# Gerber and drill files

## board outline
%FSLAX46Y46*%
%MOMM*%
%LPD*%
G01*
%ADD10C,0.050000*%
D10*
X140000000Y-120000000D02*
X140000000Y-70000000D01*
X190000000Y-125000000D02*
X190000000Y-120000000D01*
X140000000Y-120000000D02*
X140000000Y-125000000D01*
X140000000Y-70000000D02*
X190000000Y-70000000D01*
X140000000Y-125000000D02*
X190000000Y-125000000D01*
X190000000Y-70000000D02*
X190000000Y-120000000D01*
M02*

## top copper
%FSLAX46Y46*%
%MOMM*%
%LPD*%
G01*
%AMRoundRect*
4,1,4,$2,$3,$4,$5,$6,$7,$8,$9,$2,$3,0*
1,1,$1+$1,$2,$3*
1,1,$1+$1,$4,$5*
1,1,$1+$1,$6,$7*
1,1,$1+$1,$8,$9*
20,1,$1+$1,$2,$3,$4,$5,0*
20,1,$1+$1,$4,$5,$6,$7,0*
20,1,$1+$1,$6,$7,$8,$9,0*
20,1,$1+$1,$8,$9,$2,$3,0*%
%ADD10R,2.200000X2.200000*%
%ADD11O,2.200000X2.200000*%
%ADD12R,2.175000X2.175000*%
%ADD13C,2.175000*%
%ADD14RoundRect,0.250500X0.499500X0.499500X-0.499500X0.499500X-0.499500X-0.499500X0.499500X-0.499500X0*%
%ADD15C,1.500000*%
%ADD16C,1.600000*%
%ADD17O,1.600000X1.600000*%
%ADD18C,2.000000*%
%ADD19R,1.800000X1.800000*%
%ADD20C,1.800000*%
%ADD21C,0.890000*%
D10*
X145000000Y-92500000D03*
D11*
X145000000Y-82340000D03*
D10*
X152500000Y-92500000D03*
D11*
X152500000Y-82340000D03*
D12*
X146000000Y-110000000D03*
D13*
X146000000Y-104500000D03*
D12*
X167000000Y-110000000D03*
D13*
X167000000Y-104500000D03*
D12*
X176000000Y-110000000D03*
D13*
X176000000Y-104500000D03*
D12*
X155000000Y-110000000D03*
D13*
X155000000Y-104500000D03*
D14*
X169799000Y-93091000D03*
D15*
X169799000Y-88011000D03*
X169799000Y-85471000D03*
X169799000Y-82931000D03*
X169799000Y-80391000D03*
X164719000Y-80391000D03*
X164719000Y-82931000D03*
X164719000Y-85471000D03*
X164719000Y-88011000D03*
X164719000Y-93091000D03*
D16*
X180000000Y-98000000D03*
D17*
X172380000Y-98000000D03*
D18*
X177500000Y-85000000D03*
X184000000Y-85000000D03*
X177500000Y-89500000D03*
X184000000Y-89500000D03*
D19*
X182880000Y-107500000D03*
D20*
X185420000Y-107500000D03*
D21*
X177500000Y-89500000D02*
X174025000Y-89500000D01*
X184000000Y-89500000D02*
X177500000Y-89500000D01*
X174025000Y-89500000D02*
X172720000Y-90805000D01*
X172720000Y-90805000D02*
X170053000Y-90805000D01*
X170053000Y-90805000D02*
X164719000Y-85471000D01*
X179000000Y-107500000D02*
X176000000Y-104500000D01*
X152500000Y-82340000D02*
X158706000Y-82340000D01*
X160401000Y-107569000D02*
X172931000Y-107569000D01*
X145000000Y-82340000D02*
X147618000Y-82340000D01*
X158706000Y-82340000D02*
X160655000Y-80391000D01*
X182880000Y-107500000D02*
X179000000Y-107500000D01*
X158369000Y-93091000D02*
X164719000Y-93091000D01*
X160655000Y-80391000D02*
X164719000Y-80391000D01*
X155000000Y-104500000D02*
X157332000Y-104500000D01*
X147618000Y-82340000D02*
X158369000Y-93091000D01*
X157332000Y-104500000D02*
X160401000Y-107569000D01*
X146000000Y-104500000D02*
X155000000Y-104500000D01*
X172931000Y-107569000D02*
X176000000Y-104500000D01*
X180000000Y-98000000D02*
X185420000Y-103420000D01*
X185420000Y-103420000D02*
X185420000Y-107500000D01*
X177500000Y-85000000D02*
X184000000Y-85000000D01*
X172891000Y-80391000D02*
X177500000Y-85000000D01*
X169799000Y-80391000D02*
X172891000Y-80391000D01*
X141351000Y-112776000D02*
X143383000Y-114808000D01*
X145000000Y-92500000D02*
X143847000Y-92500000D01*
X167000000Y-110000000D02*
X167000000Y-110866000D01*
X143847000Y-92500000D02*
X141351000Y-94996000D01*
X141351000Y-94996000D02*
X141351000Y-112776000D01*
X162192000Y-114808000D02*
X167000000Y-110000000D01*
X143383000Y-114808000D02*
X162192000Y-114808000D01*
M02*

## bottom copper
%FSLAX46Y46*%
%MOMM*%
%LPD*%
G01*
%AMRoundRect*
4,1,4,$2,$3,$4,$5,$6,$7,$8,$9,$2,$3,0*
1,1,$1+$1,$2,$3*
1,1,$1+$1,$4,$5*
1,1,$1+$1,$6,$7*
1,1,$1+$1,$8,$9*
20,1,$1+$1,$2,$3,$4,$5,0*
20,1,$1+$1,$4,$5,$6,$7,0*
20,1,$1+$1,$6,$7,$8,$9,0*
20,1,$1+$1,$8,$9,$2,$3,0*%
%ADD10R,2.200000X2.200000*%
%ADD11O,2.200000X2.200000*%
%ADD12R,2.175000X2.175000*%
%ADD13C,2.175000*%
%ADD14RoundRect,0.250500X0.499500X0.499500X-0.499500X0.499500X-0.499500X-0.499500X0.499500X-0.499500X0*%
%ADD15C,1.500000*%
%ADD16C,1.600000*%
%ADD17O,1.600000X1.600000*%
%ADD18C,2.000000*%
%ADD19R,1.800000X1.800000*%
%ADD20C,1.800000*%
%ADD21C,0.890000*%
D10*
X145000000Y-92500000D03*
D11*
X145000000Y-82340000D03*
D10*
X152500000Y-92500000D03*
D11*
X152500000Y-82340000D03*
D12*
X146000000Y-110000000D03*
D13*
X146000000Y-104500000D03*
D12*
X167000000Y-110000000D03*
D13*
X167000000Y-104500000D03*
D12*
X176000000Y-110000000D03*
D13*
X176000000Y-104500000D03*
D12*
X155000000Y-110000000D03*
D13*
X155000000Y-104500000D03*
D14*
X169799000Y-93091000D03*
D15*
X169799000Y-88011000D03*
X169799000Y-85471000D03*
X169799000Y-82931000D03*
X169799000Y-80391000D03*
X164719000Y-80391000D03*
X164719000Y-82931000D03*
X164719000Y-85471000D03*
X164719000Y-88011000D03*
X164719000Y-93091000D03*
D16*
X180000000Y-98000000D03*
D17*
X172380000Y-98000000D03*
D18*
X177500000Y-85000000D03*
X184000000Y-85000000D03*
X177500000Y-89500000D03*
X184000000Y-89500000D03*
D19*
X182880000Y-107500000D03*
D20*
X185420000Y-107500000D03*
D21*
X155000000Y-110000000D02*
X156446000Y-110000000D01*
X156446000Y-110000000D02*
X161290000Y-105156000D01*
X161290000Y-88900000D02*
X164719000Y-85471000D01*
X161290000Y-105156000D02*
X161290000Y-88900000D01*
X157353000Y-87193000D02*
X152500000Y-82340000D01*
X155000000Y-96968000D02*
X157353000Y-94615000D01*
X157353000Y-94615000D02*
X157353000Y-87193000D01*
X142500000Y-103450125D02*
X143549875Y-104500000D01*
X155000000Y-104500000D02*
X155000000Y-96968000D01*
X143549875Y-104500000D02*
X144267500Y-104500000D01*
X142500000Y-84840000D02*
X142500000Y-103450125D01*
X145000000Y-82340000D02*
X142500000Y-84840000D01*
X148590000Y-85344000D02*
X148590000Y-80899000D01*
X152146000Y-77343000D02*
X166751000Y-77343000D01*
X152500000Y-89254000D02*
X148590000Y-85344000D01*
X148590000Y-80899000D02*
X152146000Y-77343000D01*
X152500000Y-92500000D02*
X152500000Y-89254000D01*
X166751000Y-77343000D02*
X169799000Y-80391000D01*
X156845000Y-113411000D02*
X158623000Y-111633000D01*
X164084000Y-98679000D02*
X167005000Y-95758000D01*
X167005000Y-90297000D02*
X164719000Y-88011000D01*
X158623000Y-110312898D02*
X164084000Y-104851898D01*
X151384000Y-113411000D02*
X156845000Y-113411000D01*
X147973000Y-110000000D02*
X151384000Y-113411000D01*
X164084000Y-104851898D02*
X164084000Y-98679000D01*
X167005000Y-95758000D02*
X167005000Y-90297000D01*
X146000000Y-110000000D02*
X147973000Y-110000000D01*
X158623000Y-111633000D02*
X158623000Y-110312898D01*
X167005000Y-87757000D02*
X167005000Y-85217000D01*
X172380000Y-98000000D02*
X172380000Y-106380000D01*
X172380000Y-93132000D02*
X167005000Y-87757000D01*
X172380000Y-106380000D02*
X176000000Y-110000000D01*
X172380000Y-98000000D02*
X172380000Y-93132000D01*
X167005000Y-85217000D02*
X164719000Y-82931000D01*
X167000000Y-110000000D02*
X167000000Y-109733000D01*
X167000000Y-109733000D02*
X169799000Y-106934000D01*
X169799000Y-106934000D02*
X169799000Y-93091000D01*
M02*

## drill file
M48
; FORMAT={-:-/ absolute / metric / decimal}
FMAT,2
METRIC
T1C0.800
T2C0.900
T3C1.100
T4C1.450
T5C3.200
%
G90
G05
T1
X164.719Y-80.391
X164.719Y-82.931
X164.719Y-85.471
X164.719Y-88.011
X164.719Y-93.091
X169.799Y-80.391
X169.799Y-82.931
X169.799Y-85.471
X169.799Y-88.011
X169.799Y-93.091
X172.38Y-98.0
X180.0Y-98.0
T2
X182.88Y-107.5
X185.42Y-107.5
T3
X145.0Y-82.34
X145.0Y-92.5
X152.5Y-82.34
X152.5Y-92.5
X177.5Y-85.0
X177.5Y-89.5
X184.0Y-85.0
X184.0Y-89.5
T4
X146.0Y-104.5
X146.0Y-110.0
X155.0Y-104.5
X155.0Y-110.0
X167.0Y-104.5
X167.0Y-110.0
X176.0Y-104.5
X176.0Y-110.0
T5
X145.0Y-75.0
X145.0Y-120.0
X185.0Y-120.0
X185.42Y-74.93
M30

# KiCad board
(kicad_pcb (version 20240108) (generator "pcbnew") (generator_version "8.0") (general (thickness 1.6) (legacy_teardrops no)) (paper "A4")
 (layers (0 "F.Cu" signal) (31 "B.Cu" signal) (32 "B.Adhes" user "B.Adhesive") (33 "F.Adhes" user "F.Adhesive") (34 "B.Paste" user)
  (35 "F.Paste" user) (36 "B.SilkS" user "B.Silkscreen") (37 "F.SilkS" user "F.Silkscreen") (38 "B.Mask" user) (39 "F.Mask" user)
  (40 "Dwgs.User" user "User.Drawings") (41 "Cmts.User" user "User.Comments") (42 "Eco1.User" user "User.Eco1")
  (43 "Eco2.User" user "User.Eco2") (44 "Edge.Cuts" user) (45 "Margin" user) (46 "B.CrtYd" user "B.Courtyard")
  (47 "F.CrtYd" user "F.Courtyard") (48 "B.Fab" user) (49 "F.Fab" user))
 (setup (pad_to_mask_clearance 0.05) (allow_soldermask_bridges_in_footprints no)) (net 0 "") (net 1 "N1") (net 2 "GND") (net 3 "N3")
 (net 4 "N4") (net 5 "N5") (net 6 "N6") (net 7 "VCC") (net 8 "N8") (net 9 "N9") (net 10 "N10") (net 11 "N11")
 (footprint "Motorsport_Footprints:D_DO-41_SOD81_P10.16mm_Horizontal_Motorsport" (layer "F.Cu") (at 145 92.5 90)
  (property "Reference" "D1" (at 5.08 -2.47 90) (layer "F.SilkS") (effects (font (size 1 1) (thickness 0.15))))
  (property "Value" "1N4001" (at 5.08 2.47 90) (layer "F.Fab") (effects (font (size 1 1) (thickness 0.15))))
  (pad "1" thru_hole rect (at 0 0 90) (size 2.2 2.2) (drill 1.1) (layers "*.Cu" "*.Mask") (remove_unused_layers no) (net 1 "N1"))
  (pad "2" thru_hole oval (at 10.16 0 90) (size 2.2 2.2) (drill 1.1) (layers "*.Cu" "*.Mask") (remove_unused_layers no) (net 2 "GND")))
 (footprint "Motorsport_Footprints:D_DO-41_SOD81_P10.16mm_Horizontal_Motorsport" (layer "F.Cu") (at 152.5 92.5 90)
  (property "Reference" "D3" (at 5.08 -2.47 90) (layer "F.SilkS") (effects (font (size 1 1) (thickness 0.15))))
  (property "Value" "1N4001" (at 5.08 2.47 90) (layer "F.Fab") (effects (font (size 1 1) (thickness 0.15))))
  (pad "1" thru_hole rect (at 0 0 90) (size 2.2 2.2) (drill 1.1) (layers "*.Cu" "*.Mask") (remove_unused_layers no) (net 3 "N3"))
  (pad "2" thru_hole oval (at 10.16 0 90) (size 2.2 2.2) (drill 1.1) (layers "*.Cu" "*.Mask") (remove_unused_layers no) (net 2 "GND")))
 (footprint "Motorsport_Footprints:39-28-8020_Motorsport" (layer "F.Cu") (at 146 110)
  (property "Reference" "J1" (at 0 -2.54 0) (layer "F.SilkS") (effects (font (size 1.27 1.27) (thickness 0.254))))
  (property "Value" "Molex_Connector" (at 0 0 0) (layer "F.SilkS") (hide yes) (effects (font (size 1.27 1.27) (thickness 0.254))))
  (pad "1" thru_hole rect (at 0 0) (size 2.175 2.175) (drill 1.45) (layers "*.Cu" "*.Mask") (remove_unused_layers no) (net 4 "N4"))
  (pad "2" thru_hole circle (at 0 -5.5) (size 2.175 2.175) (drill 1.45) (layers "*.Cu" "*.Mask") (remove_unused_layers no) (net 2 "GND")))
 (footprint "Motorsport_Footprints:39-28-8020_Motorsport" (layer "F.Cu") (at 167 110)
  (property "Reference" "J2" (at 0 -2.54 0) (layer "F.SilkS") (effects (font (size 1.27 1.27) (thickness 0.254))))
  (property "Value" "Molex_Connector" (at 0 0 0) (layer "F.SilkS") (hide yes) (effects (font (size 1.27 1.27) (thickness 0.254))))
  (pad "1" thru_hole rect (at 0 0) (size 2.175 2.175) (drill 1.45) (layers "*.Cu" "*.Mask") (remove_unused_layers no) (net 1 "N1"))
  (pad "2" thru_hole circle (at 0 -5.5) (size 2.175 2.175) (drill 1.45) (layers "*.Cu" "*.Mask") (remove_unused_layers no) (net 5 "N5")))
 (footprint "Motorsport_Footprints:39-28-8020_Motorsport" (layer "F.Cu") (at 176 110)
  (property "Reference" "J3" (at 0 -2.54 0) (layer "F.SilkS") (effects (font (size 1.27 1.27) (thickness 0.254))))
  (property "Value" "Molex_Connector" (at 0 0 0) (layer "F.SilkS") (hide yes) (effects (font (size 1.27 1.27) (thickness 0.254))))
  (pad "1" thru_hole rect (at 0 0) (size 2.175 2.175) (drill 1.45) (layers "*.Cu" "*.Mask") (remove_unused_layers no) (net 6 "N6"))
  (pad "2" thru_hole circle (at 0 -5.5) (size 2.175 2.175) (drill 1.45) (layers "*.Cu" "*.Mask") (remove_unused_layers no) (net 2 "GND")))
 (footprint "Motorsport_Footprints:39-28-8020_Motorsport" (layer "F.Cu") (at 155 110)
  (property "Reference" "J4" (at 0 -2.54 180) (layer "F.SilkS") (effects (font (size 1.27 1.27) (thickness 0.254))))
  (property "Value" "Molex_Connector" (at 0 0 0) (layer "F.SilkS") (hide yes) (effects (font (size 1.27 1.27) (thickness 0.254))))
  (pad "1" thru_hole rect (at 0 0) (size 2.175 2.175) (drill 1.45) (layers "*.Cu" "*.Mask") (remove_unused_layers no) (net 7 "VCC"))
  (pad "2" thru_hole circle (at 0 -5.5) (size 2.175 2.175) (drill 1.45) (layers "*.Cu" "*.Mask") (remove_unused_layers no) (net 2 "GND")))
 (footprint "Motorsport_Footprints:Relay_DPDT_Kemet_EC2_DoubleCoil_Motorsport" (layer "F.Cu") (at 165.989 85.471 180)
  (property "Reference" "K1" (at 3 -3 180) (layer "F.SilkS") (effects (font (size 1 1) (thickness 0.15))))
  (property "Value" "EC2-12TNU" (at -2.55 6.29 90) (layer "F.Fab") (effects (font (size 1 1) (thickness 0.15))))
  (pad "1" thru_hole roundrect (at -3.81 -7.62 180) (size 1.5 1.5) (drill 0.8) (layers "*.Cu" "*.Mask") (remove_unused_layers no)
   (roundrect_rratio 0.167) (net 1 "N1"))
  (pad "3" thru_hole circle (at -3.81 -2.54 180) (size 1.5 1.5) (drill 0.8) (layers "*.Cu" "*.Mask") (remove_unused_layers no) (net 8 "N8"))
  (pad "4" thru_hole circle (at -3.81 0 180) (size 1.5 1.5) (drill 0.8) (layers "*.Cu" "*.Mask") (remove_unused_layers no) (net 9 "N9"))
  (pad "5" thru_hole circle (at -3.81 2.54 180) (size 1.5 1.5) (drill 0.8) (layers "*.Cu" "*.Mask") (remove_unused_layers no) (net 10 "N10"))
  (pad "6" thru_hole circle (at -3.81 5.08 180) (size 1.5 1.5) (drill 0.8) (layers "*.Cu" "*.Mask") (remove_unused_layers no) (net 3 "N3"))
  (pad "7" thru_hole circle (at 1.27 5.08 180) (size 1.5 1.5) (drill 0.8) (layers "*.Cu" "*.Mask") (remove_unused_layers no) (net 2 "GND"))
  (pad "8" thru_hole circle (at 1.27 2.54 180) (size 1.5 1.5) (drill 0.8) (layers "*.Cu" "*.Mask") (remove_unused_layers no) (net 6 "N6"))
  (pad "9" thru_hole circle (at 1.27 0 180) (size 1.5 1.5) (drill 0.8) (layers "*.Cu" "*.Mask") (remove_unused_layers no) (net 7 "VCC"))
  (pad "10" thru_hole circle (at 1.27 -2.54 180) (size 1.5 1.5) (drill 0.8) (layers "*.Cu" "*.Mask") (remove_unused_layers no) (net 4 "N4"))
  (pad "12" thru_hole circle (at 1.27 -7.62 180) (size 1.5 1.5) (drill 0.8) (layers "*.Cu" "*.Mask") (remove_unused_layers no) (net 2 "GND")))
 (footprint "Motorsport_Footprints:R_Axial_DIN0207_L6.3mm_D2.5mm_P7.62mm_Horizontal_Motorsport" (layer "F.Cu") (at 180 98 180)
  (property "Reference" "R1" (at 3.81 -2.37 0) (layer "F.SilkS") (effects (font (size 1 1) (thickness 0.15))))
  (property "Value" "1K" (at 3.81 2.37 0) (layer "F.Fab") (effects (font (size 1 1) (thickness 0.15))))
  (pad "1" thru_hole circle (at 0 0 180) (size 1.6 1.6) (drill 0.8) (layers "*.Cu" "*.Mask") (remove_unused_layers no) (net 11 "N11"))
  (pad "2" thru_hole oval (at 7.62 0 180) (size 1.6 1.6) (drill 0.8) (layers "*.Cu" "*.Mask") (remove_unused_layers no) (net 6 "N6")))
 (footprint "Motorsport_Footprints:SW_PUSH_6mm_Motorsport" (layer "F.Cu") (at 177.5 85)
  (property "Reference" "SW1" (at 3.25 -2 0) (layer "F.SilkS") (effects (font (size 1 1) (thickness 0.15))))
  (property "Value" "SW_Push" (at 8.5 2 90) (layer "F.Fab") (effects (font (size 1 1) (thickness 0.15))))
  (pad "1" thru_hole circle (at 0 0 90) (size 2 2) (drill 1.1) (layers "*.Cu" "*.Mask") (remove_unused_layers no) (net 3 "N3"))
  (pad "1" thru_hole circle (at 6.5 0 90) (size 2 2) (drill 1.1) (layers "*.Cu" "*.Mask") (remove_unused_layers no) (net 3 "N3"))
  (pad "2" thru_hole circle (at 0 4.5 90) (size 2 2) (drill 1.1) (layers "*.Cu" "*.Mask") (remove_unused_layers no) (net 7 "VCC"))
  (pad "2" thru_hole circle (at 6.5 4.5 90) (size 2 2) (drill 1.1) (layers "*.Cu" "*.Mask") (remove_unused_layers no) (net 7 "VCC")))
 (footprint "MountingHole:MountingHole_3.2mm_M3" (layer "F.Cu") (at 185.42 74.93)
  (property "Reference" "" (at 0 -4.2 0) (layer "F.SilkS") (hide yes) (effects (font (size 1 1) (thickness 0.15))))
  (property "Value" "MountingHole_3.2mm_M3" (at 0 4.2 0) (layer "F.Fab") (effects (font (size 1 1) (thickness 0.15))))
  (pad "" np_thru_hole circle (at 0 0) (size 3.2 3.2) (drill 3.2) (layers "*.Cu" "*.Mask")))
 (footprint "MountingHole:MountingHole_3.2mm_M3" (layer "F.Cu") (at 145 75)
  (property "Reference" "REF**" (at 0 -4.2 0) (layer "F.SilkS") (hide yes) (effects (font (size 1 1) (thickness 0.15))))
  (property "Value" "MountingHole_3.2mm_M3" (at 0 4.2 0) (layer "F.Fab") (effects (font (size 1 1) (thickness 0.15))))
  (pad "" np_thru_hole circle (at 0 0) (size 3.2 3.2) (drill 3.2) (layers "*.Cu" "*.Mask")))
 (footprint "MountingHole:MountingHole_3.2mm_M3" (layer "F.Cu") (at 145 120)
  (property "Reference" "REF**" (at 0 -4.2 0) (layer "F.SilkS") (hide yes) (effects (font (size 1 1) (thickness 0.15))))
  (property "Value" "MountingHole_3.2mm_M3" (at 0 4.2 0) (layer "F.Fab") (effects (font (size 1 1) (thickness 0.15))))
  (pad "" np_thru_hole circle (at 0 0) (size 3.2 3.2) (drill 3.2) (layers "*.Cu" "*.Mask")))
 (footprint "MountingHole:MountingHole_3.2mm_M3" (layer "F.Cu") (at 185 120)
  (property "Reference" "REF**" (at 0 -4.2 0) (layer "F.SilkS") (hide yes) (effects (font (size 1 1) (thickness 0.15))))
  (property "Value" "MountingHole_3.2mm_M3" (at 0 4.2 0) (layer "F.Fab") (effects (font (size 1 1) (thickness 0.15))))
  (pad "" np_thru_hole circle (at 0 0) (size 3.2 3.2) (drill 3.2) (layers "*.Cu" "*.Mask")))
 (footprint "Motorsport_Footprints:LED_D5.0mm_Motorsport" (layer "F.Cu") (at 182.88 107.5)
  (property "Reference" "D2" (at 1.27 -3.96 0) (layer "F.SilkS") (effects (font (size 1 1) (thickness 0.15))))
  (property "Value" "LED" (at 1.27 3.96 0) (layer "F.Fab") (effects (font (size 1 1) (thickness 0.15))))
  (pad "1" thru_hole rect (at 0 0) (size 1.8 1.8) (drill 0.9) (layers "*.Cu" "*.Mask") (remove_unused_layers no) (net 2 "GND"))
  (pad "2" thru_hole circle (at 2.54 0) (size 1.8 1.8) (drill 0.9) (layers "*.Cu" "*.Mask") (remove_unused_layers no) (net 11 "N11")))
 (gr_line (start 140 120) (end 140 70) (stroke (width 0.05) (type solid)) (layer "Edge.Cuts"))
 (gr_line (start 190 125) (end 190 120) (stroke (width 0.05) (type solid)) (layer "Edge.Cuts"))
 (gr_line (start 140 120) (end 140 125) (stroke (width 0.05) (type solid)) (layer "Edge.Cuts"))
 (gr_line (start 140 70) (end 190 70) (stroke (width 0.05) (type solid)) (layer "Edge.Cuts"))
 (gr_line (start 140 125) (end 190 125) (stroke (width 0.05) (type solid)) (layer "Edge.Cuts"))
 (gr_line (start 190 70) (end 190 120) (stroke (width 0.05) (type solid)) (layer "Edge.Cuts"))
 (segment (start 177.5 89.5) (end 174.025 89.5) (width 0.89) (layer "F.Cu") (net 7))
 (segment (start 184 89.5) (end 177.5 89.5) (width 0.89) (layer "F.Cu") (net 7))
 (segment (start 174.025 89.5) (end 172.72 90.805) (width 0.89) (layer "F.Cu") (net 7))
 (segment (start 172.72 90.805) (end 170.053 90.805) (width 0.89) (layer "F.Cu") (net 7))
 (segment (start 170.053 90.805) (end 164.719 85.471) (width 0.89) (layer "F.Cu") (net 7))
 (segment (start 155 110) (end 156.446 110) (width 0.89) (layer "B.Cu") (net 7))
 (segment (start 156.446 110) (end 161.29 105.156) (width 0.89) (layer "B.Cu") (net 7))
 (segment (start 161.29 88.9) (end 164.719 85.471) (width 0.89) (layer "B.Cu") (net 7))
 (segment (start 161.29 105.156) (end 161.29 88.9) (width 0.89) (layer "B.Cu") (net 7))
 (segment (start 179 107.5) (end 176 104.5) (width 0.89) (layer "F.Cu") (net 2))
 (segment (start 152.5 82.34) (end 158.706 82.34) (width 0.89) (layer "F.Cu") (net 2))
 (segment (start 160.401 107.569) (end 172.931 107.569) (width 0.89) (layer "F.Cu") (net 2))
 (segment (start 145 82.34) (end 147.618 82.34) (width 0.89) (layer "F.Cu") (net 2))
 (segment (start 158.706 82.34) (end 160.655 80.391) (width 0.89) (layer "F.Cu") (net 2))
 (segment (start 182.88 107.5) (end 179 107.5) (width 0.89) (layer "F.Cu") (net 2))
 (segment (start 158.369 93.091) (end 164.719 93.091) (width 0.89) (layer "F.Cu") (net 2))
 (segment (start 160.655 80.391) (end 164.719 80.391) (width 0.89) (layer "F.Cu") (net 2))
 (segment (start 155 104.5) (end 157.332 104.5) (width 0.89) (layer "F.Cu") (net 2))
 (segment (start 147.618 82.34) (end 158.369 93.091) (width 0.89) (layer "F.Cu") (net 2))
 (segment (start 157.332 104.5) (end 160.401 107.569) (width 0.89) (layer "F.Cu") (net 2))
 (segment (start 146 104.5) (end 155 104.5) (width 0.89) (layer "F.Cu") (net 2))
 (segment (start 172.931 107.569) (end 176 104.5) (width 0.89) (layer "F.Cu") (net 2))
 (segment (start 157.353 87.193) (end 152.5 82.34) (width 0.89) (layer "B.Cu") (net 2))
 (segment (start 155 96.968) (end 157.353 94.615) (width 0.89) (layer "B.Cu") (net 2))
 (segment (start 157.353 94.615) (end 157.353 87.193) (width 0.89) (layer "B.Cu") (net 2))
 (segment (start 142.5 103.450125) (end 143.549875 104.5) (width 0.89) (layer "B.Cu") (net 2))
 (segment (start 155 104.5) (end 155 96.968) (width 0.89) (layer "B.Cu") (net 2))
 (segment (start 143.549875 104.5) (end 144.2675 104.5) (width 0.89) (layer "B.Cu") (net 2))
 (segment (start 142.5 84.84) (end 142.5 103.450125) (width 0.89) (layer "B.Cu") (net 2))
 (segment (start 145 82.34) (end 142.5 84.84) (width 0.89) (layer "B.Cu") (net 2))
 (segment (start 180 98) (end 185.42 103.42) (width 0.89) (layer "F.Cu") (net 11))
 (segment (start 185.42 103.42) (end 185.42 107.5) (width 0.89) (layer "F.Cu") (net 11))
 (segment (start 177.5 85) (end 184 85) (width 0.89) (layer "F.Cu") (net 3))
 (segment (start 172.891 80.391) (end 177.5 85) (width 0.89) (layer "F.Cu") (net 3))
 (segment (start 169.799 80.391) (end 172.891 80.391) (width 0.89) (layer "F.Cu") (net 3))
 (segment (start 148.59 85.344) (end 148.59 80.899) (width 0.89) (layer "B.Cu") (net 3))
 (segment (start 152.146 77.343) (end 166.751 77.343) (width 0.89) (layer "B.Cu") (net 3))
 (segment (start 152.5 89.254) (end 148.59 85.344) (width 0.89) (layer "B.Cu") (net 3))
 (segment (start 148.59 80.899) (end 152.146 77.343) (width 0.89) (layer "B.Cu") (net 3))
 (segment (start 152.5 92.5) (end 152.5 89.254) (width 0.89) (layer "B.Cu") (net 3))
 (segment (start 166.751 77.343) (end 169.799 80.391) (width 0.89) (layer "B.Cu") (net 3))
 (segment (start 156.845 113.411) (end 158.623 111.633) (width 0.89) (layer "B.Cu") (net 4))
 (segment (start 164.084 98.679) (end 167.005 95.758) (width 0.89) (layer "B.Cu") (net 4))
 (segment (start 167.005 90.297) (end 164.719 88.011) (width 0.89) (layer "B.Cu") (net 4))
 (segment (start 158.623 110.312898) (end 164.084 104.851898) (width 0.89) (layer "B.Cu") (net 4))
 (segment (start 151.384 113.411) (end 156.845 113.411) (width 0.89) (layer "B.Cu") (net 4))
 (segment (start 147.973 110) (end 151.384 113.411) (width 0.89) (layer "B.Cu") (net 4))
 (segment (start 164.084 104.851898) (end 164.084 98.679) (width 0.89) (layer "B.Cu") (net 4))
 (segment (start 167.005 95.758) (end 167.005 90.297) (width 0.89) (layer "B.Cu") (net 4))
 (segment (start 146 110) (end 147.973 110) (width 0.89) (layer "B.Cu") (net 4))
 (segment (start 158.623 111.633) (end 158.623 110.312898) (width 0.89) (layer "B.Cu") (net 4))
 (segment (start 167.005 87.757) (end 167.005 85.217) (width 0.89) (layer "B.Cu") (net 6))
 (segment (start 172.38 98) (end 172.38 106.38) (width 0.89) (layer "B.Cu") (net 6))
 (segment (start 172.38 93.132) (end 167.005 87.757) (width 0.89) (layer "B.Cu") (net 6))
 (segment (start 172.38 106.38) (end 176 110) (width 0.89) (layer "B.Cu") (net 6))
 (segment (start 172.38 98) (end 172.38 93.132) (width 0.89) (layer "B.Cu") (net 6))
 (segment (start 167.005 85.217) (end 164.719 82.931) (width 0.89) (layer "B.Cu") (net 6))
 (segment (start 141.351 112.776) (end 143.383 114.808) (width 0.89) (layer "F.Cu") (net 1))
 (segment (start 145 92.5) (end 143.847 92.5) (width 0.89) (layer "F.Cu") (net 1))
 (segment (start 167 110) (end 167 110.866) (width 0.89) (layer "F.Cu") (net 1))
 (segment (start 143.847 92.5) (end 141.351 94.996) (width 0.89) (layer "F.Cu") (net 1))
 (segment (start 141.351 94.996) (end 141.351 112.776) (width 0.89) (layer "F.Cu") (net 1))
 (segment (start 162.192 114.808) (end 167 110) (width 0.89) (layer "F.Cu") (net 1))
 (segment (start 143.383 114.808) (end 162.192 114.808) (width 0.89) (layer "F.Cu") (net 1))
 (segment (start 167 110) (end 167 109.733) (width 0.89) (layer "B.Cu") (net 1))
 (segment (start 167 109.733) (end 169.799 106.934) (width 0.89) (layer "B.Cu") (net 1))
 (segment (start 169.799 106.934) (end 169.799 93.091) (width 0.89) (layer "B.Cu") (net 1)))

